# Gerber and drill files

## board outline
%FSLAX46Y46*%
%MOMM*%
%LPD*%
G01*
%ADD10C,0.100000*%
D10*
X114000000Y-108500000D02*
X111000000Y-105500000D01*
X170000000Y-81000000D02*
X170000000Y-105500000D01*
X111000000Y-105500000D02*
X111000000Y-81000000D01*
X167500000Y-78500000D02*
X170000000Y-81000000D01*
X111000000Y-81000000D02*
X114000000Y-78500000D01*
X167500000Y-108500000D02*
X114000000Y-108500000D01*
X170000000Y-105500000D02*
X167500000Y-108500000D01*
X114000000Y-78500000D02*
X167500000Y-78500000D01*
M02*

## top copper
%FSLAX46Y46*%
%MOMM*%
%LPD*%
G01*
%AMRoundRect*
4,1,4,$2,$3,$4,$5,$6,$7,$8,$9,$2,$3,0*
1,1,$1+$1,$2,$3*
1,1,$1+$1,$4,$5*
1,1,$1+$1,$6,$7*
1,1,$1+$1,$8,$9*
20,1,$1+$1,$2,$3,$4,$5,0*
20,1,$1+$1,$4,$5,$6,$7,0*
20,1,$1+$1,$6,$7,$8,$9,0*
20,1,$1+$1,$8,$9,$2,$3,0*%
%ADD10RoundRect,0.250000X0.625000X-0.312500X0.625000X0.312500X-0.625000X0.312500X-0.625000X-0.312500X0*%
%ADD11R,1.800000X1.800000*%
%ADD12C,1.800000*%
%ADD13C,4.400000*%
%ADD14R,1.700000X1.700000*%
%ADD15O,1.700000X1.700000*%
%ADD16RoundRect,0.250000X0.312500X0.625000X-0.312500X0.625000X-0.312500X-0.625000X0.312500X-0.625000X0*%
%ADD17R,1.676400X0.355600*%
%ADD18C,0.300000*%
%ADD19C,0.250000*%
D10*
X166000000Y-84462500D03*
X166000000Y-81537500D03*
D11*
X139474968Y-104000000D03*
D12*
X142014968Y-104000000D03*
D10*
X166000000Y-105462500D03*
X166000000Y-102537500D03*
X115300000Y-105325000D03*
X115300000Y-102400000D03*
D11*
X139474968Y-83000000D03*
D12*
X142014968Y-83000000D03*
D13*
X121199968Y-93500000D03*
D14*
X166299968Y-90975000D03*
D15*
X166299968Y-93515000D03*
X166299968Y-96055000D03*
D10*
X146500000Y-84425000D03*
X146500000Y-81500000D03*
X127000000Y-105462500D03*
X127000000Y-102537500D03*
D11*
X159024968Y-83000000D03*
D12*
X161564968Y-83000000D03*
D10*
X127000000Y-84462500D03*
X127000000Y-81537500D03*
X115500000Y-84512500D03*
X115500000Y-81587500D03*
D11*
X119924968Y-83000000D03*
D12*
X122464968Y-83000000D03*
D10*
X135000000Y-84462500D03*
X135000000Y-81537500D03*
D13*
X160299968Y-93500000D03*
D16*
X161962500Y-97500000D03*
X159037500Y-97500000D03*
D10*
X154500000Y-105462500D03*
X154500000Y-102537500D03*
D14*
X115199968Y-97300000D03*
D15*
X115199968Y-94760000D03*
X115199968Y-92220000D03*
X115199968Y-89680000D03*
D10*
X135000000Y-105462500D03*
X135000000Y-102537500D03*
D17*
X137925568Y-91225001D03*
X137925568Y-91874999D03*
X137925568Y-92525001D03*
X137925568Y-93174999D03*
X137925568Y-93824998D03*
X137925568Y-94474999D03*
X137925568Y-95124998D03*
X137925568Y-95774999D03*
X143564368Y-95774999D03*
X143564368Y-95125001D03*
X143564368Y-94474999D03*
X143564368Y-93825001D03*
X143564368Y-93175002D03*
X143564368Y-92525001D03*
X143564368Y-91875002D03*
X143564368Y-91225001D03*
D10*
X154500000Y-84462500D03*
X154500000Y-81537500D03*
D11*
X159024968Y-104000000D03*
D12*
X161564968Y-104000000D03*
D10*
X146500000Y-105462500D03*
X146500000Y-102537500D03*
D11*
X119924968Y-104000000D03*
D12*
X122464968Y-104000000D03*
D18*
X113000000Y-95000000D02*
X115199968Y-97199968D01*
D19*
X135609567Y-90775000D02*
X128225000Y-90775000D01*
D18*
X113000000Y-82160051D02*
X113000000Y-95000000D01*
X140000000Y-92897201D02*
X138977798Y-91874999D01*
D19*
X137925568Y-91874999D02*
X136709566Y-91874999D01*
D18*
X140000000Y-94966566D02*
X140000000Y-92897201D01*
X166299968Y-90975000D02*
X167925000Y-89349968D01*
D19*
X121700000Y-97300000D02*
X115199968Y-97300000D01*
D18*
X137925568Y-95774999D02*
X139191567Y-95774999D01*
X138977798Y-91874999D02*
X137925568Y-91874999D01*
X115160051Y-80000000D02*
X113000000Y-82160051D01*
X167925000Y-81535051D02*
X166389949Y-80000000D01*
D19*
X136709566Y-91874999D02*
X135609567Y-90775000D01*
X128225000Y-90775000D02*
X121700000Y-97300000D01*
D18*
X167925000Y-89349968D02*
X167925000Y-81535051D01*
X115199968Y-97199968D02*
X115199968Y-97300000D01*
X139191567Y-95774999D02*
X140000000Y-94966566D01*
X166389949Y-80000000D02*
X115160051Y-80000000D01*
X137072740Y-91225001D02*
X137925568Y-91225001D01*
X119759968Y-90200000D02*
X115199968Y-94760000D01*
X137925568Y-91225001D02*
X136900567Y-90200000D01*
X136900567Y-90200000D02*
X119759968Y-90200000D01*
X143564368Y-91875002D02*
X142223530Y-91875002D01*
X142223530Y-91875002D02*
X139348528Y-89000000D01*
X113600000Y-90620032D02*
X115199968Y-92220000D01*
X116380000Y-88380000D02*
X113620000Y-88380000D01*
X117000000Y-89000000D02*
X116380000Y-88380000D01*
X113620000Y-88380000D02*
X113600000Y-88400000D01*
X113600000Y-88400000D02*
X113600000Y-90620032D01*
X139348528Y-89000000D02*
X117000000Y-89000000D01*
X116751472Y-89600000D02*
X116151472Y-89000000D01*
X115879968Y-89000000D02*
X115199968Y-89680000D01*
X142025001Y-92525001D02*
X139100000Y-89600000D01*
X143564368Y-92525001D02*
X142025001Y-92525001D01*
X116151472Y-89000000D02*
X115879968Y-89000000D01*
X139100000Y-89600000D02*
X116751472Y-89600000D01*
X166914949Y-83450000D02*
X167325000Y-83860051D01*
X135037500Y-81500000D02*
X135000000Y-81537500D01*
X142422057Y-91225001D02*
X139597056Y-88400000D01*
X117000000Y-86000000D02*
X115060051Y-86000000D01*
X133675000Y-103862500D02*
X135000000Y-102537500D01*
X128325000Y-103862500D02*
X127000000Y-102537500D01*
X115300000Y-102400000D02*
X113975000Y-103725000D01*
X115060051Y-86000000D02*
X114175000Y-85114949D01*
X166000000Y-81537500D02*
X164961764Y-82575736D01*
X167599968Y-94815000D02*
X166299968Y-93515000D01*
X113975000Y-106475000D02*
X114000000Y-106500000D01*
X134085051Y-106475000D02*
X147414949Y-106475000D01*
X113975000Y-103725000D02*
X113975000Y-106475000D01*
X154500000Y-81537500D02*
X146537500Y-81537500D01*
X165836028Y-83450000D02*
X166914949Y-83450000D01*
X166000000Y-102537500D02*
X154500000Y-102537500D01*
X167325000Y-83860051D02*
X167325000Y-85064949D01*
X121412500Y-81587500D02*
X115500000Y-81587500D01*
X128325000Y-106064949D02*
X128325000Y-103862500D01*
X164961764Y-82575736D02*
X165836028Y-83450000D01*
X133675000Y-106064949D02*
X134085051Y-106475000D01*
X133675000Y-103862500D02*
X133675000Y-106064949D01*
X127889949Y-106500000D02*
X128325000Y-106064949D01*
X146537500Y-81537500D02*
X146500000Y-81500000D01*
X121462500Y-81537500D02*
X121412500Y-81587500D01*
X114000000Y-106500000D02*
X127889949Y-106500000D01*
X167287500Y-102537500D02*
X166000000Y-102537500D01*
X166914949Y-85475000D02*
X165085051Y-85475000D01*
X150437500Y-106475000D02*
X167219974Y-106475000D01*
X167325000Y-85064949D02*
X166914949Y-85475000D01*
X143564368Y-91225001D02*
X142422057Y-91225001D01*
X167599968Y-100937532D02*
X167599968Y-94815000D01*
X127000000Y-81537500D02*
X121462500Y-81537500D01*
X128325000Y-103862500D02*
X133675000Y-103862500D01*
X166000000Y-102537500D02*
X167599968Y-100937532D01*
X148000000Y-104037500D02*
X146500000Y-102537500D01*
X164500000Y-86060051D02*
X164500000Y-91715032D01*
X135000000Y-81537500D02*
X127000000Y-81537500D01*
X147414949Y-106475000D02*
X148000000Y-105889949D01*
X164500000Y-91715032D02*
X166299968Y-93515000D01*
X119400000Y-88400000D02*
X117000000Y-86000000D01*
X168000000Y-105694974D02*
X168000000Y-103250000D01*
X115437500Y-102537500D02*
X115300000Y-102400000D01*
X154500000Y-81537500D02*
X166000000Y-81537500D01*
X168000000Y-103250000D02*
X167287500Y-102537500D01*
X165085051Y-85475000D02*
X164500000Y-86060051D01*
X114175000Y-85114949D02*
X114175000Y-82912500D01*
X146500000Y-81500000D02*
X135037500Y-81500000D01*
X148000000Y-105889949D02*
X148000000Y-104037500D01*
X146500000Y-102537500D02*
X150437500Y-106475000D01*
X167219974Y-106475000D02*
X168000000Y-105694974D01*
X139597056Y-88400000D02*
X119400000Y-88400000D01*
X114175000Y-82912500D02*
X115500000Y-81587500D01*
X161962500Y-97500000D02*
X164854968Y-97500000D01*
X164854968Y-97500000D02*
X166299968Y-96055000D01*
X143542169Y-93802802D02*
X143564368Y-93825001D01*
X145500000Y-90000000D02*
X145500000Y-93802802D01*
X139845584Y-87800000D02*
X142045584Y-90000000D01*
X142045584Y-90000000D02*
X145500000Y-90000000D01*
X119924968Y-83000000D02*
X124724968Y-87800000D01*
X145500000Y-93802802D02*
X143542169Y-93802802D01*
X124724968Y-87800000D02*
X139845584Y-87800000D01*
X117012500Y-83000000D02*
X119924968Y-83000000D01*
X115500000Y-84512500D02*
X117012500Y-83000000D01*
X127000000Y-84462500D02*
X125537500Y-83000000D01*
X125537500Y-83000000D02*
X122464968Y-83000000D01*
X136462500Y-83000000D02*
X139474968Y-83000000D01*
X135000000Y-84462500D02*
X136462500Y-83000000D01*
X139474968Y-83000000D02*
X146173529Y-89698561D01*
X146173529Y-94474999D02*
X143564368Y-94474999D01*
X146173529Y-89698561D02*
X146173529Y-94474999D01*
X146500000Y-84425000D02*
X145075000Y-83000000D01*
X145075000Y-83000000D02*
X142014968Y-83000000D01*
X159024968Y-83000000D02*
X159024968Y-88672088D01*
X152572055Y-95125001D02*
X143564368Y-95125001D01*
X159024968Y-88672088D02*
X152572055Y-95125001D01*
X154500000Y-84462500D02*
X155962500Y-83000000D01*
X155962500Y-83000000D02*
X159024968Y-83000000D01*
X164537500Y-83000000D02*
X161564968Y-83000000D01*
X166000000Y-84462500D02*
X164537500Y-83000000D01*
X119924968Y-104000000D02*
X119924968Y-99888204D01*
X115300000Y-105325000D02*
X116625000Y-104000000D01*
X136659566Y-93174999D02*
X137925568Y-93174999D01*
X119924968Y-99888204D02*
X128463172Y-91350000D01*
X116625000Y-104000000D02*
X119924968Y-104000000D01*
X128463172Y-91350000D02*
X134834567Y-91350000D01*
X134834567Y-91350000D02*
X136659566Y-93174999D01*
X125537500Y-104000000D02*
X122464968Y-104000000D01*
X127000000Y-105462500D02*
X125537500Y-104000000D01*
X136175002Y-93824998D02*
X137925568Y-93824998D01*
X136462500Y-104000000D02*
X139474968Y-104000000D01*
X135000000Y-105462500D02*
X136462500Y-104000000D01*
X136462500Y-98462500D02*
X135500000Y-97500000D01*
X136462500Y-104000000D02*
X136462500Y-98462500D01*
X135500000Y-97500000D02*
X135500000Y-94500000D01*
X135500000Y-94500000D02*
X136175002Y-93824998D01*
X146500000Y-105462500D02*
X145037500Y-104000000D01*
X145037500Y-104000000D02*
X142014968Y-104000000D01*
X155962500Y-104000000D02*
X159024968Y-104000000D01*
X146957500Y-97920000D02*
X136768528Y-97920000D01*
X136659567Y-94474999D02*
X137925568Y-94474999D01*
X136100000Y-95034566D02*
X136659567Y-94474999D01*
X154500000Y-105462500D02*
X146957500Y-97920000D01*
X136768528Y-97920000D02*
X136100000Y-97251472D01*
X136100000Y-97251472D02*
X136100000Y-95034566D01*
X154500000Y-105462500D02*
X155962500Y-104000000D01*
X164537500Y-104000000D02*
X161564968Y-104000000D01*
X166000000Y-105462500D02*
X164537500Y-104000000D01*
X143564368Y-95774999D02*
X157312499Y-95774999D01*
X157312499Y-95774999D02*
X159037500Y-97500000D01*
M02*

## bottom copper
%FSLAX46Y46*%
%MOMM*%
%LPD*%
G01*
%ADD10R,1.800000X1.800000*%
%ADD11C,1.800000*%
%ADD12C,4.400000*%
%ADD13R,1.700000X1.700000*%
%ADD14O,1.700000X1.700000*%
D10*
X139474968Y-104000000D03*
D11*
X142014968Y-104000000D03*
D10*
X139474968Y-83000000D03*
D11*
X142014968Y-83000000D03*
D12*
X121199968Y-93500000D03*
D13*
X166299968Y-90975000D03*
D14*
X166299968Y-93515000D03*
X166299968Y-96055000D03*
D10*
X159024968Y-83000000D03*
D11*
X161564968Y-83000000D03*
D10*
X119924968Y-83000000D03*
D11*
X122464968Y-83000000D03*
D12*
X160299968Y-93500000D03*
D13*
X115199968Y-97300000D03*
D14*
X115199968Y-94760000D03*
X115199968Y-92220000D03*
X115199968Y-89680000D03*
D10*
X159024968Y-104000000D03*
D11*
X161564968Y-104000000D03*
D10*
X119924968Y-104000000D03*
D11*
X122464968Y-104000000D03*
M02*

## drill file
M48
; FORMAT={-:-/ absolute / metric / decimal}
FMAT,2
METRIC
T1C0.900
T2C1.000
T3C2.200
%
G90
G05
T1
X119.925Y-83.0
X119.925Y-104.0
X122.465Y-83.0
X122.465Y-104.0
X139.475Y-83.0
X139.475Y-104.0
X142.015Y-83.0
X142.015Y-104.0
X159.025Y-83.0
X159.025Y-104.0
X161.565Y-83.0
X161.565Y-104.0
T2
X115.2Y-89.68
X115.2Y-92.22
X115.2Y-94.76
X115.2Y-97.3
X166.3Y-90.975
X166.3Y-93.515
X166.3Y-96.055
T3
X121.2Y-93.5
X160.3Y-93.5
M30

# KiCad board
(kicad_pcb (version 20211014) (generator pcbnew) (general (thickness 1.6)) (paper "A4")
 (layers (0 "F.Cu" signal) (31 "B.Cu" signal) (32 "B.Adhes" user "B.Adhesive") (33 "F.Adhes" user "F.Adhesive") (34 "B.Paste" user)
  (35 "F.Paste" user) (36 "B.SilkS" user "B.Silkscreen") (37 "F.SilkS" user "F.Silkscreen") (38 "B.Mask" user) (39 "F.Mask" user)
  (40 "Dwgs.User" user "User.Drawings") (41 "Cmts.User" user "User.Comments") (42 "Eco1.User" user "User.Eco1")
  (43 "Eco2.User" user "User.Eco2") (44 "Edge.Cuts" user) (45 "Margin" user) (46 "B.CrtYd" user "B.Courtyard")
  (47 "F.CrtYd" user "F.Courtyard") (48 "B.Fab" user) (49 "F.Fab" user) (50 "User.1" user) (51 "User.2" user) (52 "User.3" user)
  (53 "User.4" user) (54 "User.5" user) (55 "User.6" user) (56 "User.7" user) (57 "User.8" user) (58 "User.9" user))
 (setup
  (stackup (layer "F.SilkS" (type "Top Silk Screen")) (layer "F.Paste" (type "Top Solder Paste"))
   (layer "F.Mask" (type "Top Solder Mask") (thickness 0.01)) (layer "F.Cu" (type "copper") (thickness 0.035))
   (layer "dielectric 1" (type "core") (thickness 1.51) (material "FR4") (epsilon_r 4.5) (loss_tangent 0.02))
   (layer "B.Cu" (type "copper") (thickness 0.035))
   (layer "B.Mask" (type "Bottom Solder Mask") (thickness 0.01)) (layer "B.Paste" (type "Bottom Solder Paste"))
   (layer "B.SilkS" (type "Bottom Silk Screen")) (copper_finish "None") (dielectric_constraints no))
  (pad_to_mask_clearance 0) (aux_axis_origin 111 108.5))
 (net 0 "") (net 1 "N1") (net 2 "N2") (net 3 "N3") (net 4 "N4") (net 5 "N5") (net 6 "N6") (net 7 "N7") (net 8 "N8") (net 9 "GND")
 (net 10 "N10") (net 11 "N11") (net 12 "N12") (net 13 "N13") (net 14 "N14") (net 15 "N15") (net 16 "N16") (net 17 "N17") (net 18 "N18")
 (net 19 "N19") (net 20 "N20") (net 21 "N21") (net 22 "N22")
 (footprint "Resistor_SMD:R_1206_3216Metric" (layer "F.Cu") (at 166 83 90)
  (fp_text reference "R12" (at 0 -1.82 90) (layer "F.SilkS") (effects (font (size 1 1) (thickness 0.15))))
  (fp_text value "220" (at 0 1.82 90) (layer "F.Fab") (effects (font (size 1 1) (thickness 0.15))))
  (pad "1" smd roundrect (at -1.4625 0 90) (size 1.125 1.75) (layers "F.Cu" "F.Paste" "F.Mask") (roundrect_rratio 0.2222222222) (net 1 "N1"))
  (pad "2" smd roundrect (at 1.4625 0 90) (size 1.125 1.75) (layers "F.Cu" "F.Paste" "F.Mask") (roundrect_rratio 0.2222222222) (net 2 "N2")))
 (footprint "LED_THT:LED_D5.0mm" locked (layer "F.Cu") (at 139.474968 104)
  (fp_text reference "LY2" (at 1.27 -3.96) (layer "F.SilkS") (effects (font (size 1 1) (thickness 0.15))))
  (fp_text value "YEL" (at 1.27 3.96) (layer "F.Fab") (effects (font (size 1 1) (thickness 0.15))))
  (pad "1" thru_hole rect locked (at 0 0) (size 1.8 1.8) (drill 0.9) (layers *.Cu *.Mask) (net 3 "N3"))
  (pad "2" thru_hole circle locked (at 2.54 0) (size 1.8 1.8) (drill 0.9) (layers *.Cu *.Mask) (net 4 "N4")))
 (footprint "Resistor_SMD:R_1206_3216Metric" (layer "F.Cu") (at 166 104 90)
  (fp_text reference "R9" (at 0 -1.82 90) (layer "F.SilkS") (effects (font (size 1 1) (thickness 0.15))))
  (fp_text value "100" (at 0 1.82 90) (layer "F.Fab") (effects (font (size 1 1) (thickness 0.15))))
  (pad "1" smd roundrect (at -1.4625 0 90) (size 1.125 1.75) (layers "F.Cu" "F.Paste" "F.Mask") (roundrect_rratio 0.2222222222) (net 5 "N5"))
  (pad "2" smd roundrect (at 1.4625 0 90) (size 1.125 1.75) (layers "F.Cu" "F.Paste" "F.Mask") (roundrect_rratio 0.2222222222) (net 2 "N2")))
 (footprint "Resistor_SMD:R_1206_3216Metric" (layer "F.Cu") (at 115.3 103.8625 90)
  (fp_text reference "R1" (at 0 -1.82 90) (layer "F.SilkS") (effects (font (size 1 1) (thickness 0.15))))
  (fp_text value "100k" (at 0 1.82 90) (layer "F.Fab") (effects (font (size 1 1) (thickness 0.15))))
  (pad "1" smd roundrect (at -1.4625 0 90) (size 1.125 1.75) (layers "F.Cu" "F.Paste" "F.Mask") (roundrect_rratio 0.2222222222) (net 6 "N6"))
  (pad "2" smd roundrect (at 1.4625 0 90) (size 1.125 1.75) (layers "F.Cu" "F.Paste" "F.Mask") (roundrect_rratio 0.2222222222) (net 2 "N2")))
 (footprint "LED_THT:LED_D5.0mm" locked (layer "F.Cu") (at 139.474968 83)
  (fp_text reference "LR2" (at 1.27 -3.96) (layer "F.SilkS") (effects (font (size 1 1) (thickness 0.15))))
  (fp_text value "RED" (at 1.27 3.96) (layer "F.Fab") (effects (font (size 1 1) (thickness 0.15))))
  (pad "1" thru_hole rect locked (at 0 0) (size 1.8 1.8) (drill 0.9) (layers *.Cu *.Mask) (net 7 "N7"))
  (pad "2" thru_hole circle locked (at 2.54 0) (size 1.8 1.8) (drill 0.9) (layers *.Cu *.Mask) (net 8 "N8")))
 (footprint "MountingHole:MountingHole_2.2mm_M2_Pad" (layer "F.Cu") (at 121.199968 93.5)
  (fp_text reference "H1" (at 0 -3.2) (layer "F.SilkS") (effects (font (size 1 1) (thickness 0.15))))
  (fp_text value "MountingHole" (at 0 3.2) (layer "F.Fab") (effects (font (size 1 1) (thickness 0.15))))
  (pad "1" thru_hole circle (at 0 0) (size 4.4 4.4) (drill 2.2) (layers *.Cu *.Mask)))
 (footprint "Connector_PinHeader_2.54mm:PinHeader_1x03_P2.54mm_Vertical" (layer "F.Cu") (at 166.299968 90.975)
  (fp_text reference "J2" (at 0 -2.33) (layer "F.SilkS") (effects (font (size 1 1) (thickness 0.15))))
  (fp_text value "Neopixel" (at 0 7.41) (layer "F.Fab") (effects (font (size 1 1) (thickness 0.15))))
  (pad "1" thru_hole rect (at 0 0) (size 1.7 1.7) (drill 1) (layers *.Cu *.Mask) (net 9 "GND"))
  (pad "2" thru_hole oval (at 0 2.54) (size 1.7 1.7) (drill 1) (layers *.Cu *.Mask) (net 2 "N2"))
  (pad "3" thru_hole oval (at 0 5.08) (size 1.7 1.7) (drill 1) (layers *.Cu *.Mask) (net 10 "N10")))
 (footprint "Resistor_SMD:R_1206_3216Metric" (layer "F.Cu") (at 146.5 82.9625 90)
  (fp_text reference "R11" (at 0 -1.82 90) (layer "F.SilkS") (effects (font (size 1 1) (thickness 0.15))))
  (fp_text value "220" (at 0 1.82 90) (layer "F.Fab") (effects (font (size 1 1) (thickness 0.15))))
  (pad "1" smd roundrect (at -1.4625 0 90) (size 1.125 1.75) (layers "F.Cu" "F.Paste" "F.Mask") (roundrect_rratio 0.2222222222) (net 8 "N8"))
  (pad "2" smd roundrect (at 1.4625 0 90) (size 1.125 1.75) (layers "F.Cu" "F.Paste" "F.Mask") (roundrect_rratio 0.2222222222) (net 2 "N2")))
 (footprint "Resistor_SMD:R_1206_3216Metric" (layer "F.Cu") (at 127 104 90)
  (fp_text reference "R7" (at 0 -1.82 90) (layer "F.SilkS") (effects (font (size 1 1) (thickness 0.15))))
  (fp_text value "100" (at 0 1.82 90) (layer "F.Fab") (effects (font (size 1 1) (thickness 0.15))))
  (pad "1" smd roundrect (at -1.4625 0 90) (size 1.125 1.75) (layers "F.Cu" "F.Paste" "F.Mask") (roundrect_rratio 0.2222222222)
   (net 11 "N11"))
  (pad "2" smd roundrect (at 1.4625 0 90) (size 1.125 1.75) (layers "F.Cu" "F.Paste" "F.Mask") (roundrect_rratio 0.2222222222) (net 2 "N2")))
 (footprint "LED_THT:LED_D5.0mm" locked (layer "F.Cu") (at 159.024968 83)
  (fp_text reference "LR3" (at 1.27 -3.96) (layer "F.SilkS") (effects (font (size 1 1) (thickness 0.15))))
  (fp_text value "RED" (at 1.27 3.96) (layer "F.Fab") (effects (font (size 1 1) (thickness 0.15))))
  (pad "1" thru_hole rect locked (at 0 0) (size 1.8 1.8) (drill 0.9) (layers *.Cu *.Mask) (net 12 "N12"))
  (pad "2" thru_hole circle locked (at 2.54 0) (size 1.8 1.8) (drill 0.9) (layers *.Cu *.Mask) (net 1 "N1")))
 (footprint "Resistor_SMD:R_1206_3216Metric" (layer "F.Cu") (at 127 83 90)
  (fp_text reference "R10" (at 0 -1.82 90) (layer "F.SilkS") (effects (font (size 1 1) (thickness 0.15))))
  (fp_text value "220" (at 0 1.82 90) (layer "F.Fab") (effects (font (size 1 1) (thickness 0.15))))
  (pad "1" smd roundrect (at -1.4625 0 90) (size 1.125 1.75) (layers "F.Cu" "F.Paste" "F.Mask") (roundrect_rratio 0.2222222222)
   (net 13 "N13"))
  (pad "2" smd roundrect (at 1.4625 0 90) (size 1.125 1.75) (layers "F.Cu" "F.Paste" "F.Mask") (roundrect_rratio 0.2222222222) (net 2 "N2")))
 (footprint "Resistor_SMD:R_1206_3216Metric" (layer "F.Cu") (at 115.5 83.05 90)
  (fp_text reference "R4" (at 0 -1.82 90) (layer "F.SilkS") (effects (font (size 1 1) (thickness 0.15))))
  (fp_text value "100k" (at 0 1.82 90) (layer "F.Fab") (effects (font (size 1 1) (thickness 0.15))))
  (pad "1" smd roundrect (at -1.4625 0 90) (size 1.125 1.75) (layers "F.Cu" "F.Paste" "F.Mask") (roundrect_rratio 0.2222222222)
   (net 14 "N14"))
  (pad "2" smd roundrect (at 1.4625 0 90) (size 1.125 1.75) (layers "F.Cu" "F.Paste" "F.Mask") (roundrect_rratio 0.2222222222) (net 2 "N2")))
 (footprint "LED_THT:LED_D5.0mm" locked (layer "F.Cu") (at 119.924968 83)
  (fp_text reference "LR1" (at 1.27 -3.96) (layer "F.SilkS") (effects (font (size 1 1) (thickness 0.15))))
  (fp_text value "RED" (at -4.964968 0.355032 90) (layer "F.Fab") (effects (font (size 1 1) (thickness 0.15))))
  (pad "1" thru_hole rect locked (at 0 0) (size 1.8 1.8) (drill 0.9) (layers *.Cu *.Mask) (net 14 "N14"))
  (pad "2" thru_hole circle locked (at 2.54 0) (size 1.8 1.8) (drill 0.9) (layers *.Cu *.Mask) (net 13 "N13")))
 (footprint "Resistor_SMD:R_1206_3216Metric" (layer "F.Cu") (at 135 83 90)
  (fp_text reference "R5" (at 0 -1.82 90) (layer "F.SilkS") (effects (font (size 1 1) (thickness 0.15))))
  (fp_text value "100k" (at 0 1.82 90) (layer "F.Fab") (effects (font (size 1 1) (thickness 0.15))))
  (pad "1" smd roundrect (at -1.4625 0 90) (size 1.125 1.75) (layers "F.Cu" "F.Paste" "F.Mask") (roundrect_rratio 0.2222222222) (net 7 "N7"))
  (pad "2" smd roundrect (at 1.4625 0 90) (size 1.125 1.75) (layers "F.Cu" "F.Paste" "F.Mask") (roundrect_rratio 0.2222222222) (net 2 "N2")))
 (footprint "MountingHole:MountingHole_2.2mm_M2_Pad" (layer "F.Cu") (at 160.299968 93.5)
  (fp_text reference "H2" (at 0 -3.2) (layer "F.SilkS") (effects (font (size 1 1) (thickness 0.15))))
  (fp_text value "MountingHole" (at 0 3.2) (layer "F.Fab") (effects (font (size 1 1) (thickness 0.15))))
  (pad "1" thru_hole circle (at 0 0) (size 4.4 4.4) (drill 2.2) (layers *.Cu *.Mask)))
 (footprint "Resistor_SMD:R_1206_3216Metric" (layer "F.Cu") (at 160.5 97.5 180)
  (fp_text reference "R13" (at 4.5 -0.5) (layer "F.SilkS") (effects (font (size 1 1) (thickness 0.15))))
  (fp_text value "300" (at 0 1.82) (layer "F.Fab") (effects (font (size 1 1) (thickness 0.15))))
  (pad "1" smd roundrect (at -1.4625 0 180) (size 1.125 1.75) (layers "F.Cu" "F.Paste" "F.Mask") (roundrect_rratio 0.2222222222)
   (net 10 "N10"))
  (pad "2" smd roundrect (at 1.4625 0 180) (size 1.125 1.75) (layers "F.Cu" "F.Paste" "F.Mask") (roundrect_rratio 0.2222222222)
   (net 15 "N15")))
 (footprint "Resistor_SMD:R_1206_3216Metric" (layer "F.Cu") (at 154.5 104 90)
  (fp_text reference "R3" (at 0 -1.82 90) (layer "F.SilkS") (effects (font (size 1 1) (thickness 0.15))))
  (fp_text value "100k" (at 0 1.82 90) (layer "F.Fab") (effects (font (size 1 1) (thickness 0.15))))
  (pad "1" smd roundrect (at -1.4625 0 90) (size 1.125 1.75) (layers "F.Cu" "F.Paste" "F.Mask") (roundrect_rratio 0.2222222222)
   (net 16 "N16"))
  (pad "2" smd roundrect (at 1.4625 0 90) (size 1.125 1.75) (layers "F.Cu" "F.Paste" "F.Mask") (roundrect_rratio 0.2222222222) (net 2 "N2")))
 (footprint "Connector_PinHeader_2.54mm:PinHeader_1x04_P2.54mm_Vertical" (layer "F.Cu") (at 115.199968 97.3 180)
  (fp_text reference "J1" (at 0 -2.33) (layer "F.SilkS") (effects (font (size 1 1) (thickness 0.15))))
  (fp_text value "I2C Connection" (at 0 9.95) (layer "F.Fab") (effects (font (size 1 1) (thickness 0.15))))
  (pad "1" thru_hole rect (at 0 0 180) (size 1.7 1.7) (drill 1) (layers *.Cu *.Mask) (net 9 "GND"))
  (pad "2" thru_hole oval (at 0 2.54 180) (size 1.7 1.7) (drill 1) (layers *.Cu *.Mask) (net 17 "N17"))
  (pad "3" thru_hole oval (at 0 5.08 180) (size 1.7 1.7) (drill 1) (layers *.Cu *.Mask) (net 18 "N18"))
  (pad "4" thru_hole oval (at 0 7.62 180) (size 1.7 1.7) (drill 1) (layers *.Cu *.Mask) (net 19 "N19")))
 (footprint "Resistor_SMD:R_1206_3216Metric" (layer "F.Cu") (at 135 104 90)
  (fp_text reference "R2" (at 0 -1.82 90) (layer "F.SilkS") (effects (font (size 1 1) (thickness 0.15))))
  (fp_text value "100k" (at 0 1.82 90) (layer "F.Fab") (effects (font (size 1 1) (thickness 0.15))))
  (pad "1" smd roundrect (at -1.4625 0 90) (size 1.125 1.75) (layers "F.Cu" "F.Paste" "F.Mask") (roundrect_rratio 0.2222222222) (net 3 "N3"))
  (pad "2" smd roundrect (at 1.4625 0 90) (size 1.125 1.75) (layers "F.Cu" "F.Paste" "F.Mask") (roundrect_rratio 0.2222222222) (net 2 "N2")))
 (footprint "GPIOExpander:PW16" (layer "F.Cu") (at 140.744968 93.5)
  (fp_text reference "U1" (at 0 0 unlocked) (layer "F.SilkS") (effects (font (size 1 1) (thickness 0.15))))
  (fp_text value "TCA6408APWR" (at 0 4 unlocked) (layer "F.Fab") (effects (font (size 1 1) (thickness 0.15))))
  (pad "1" smd rect (at -2.8194 -2.274999) (size 1.6764 0.3556) (layers "F.Cu" "F.Paste" "F.Mask") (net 17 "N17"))
  (pad "2" smd rect (at -2.8194 -1.625001) (size 1.6764 0.3556) (layers "F.Cu" "F.Paste" "F.Mask") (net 9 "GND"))
  (pad "3" smd rect (at -2.8194 -0.974999) (size 1.6764 0.3556) (layers "F.Cu" "F.Paste" "F.Mask") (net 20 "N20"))
  (pad "4" smd rect (at -2.8194 -0.325001) (size 1.6764 0.3556) (layers "F.Cu" "F.Paste" "F.Mask") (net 6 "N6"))
  (pad "5" smd rect (at -2.8194 0.324998) (size 1.6764 0.3556) (layers "F.Cu" "F.Paste" "F.Mask") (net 3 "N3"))
  (pad "6" smd rect (at -2.8194 0.974999) (size 1.6764 0.3556) (layers "F.Cu" "F.Paste" "F.Mask") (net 16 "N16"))
  (pad "7" smd rect (at -2.8194 1.624998) (size 1.6764 0.3556) (layers "F.Cu" "F.Paste" "F.Mask") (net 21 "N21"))
  (pad "8" smd rect (at -2.8194 2.274999) (size 1.6764 0.3556) (layers "F.Cu" "F.Paste" "F.Mask") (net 9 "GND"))
  (pad "9" smd rect (at 2.8194 2.274999) (size 1.6764 0.3556) (layers "F.Cu" "F.Paste" "F.Mask") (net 15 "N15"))
  (pad "10" smd rect (at 2.8194 1.625001) (size 1.6764 0.3556) (layers "F.Cu" "F.Paste" "F.Mask") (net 12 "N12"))
  (pad "11" smd rect (at 2.8194 0.974999) (size 1.6764 0.3556) (layers "F.Cu" "F.Paste" "F.Mask") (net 7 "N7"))
  (pad "12" smd rect (at 2.8194 0.325001) (size 1.6764 0.3556) (layers "F.Cu" "F.Paste" "F.Mask") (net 14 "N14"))
  (pad "13" smd rect (at 2.8194 -0.324998) (size 1.6764 0.3556) (layers "F.Cu" "F.Paste" "F.Mask") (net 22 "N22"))
  (pad "14" smd rect (at 2.8194 -0.974999) (size 1.6764 0.3556) (layers "F.Cu" "F.Paste" "F.Mask") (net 19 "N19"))
  (pad "15" smd rect (at 2.8194 -1.624998) (size 1.6764 0.3556) (layers "F.Cu" "F.Paste" "F.Mask") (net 18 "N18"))
  (pad "16" smd rect (at 2.8194 -2.274999) (size 1.6764 0.3556) (layers "F.Cu" "F.Paste" "F.Mask") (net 2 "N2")))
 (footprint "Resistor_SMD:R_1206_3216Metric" (layer "F.Cu") (at 154.5 83 90)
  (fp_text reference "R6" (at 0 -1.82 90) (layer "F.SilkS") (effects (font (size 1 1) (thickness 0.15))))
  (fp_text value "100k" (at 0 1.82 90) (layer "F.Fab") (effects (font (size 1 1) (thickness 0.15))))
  (pad "1" smd roundrect (at -1.4625 0 90) (size 1.125 1.75) (layers "F.Cu" "F.Paste" "F.Mask") (roundrect_rratio 0.2222222222)
   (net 12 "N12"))
  (pad "2" smd roundrect (at 1.4625 0 90) (size 1.125 1.75) (layers "F.Cu" "F.Paste" "F.Mask") (roundrect_rratio 0.2222222222) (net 2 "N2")))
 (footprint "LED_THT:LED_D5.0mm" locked (layer "F.Cu") (at 159.024968 104)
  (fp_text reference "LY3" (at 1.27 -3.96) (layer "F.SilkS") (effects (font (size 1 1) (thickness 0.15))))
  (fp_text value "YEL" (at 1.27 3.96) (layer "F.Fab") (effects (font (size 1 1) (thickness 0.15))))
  (pad "1" thru_hole rect locked (at 0 0) (size 1.8 1.8) (drill 0.9) (layers *.Cu *.Mask) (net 16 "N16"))
  (pad "2" thru_hole circle locked (at 2.54 0) (size 1.8 1.8) (drill 0.9) (layers *.Cu *.Mask) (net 5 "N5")))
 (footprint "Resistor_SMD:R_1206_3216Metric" (layer "F.Cu") (at 146.5 104 90)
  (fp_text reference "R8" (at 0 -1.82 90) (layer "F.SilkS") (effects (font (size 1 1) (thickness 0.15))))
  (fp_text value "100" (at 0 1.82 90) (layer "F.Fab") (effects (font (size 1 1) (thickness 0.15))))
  (pad "1" smd roundrect (at -1.4625 0 90) (size 1.125 1.75) (layers "F.Cu" "F.Paste" "F.Mask") (roundrect_rratio 0.2222222222) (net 4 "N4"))
  (pad "2" smd roundrect (at 1.4625 0 90) (size 1.125 1.75) (layers "F.Cu" "F.Paste" "F.Mask") (roundrect_rratio 0.2222222222) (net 2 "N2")))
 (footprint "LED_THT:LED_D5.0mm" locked (layer "F.Cu") (at 119.924968 104)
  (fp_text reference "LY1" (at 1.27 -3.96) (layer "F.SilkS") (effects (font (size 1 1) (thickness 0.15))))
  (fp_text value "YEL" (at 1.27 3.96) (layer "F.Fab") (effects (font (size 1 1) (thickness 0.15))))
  (pad "1" thru_hole rect locked (at 0 0) (size 1.8 1.8) (drill 0.9) (layers *.Cu *.Mask) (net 6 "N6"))
  (pad "2" thru_hole circle locked (at 2.54 0) (size 1.8 1.8) (drill 0.9) (layers *.Cu *.Mask) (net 11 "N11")))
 (gr_line (start 114 108.5) (end 111 105.5) (layer "Edge.Cuts") (width 0.1))
 (gr_line (start 170 81) (end 170 105.5) (layer "Edge.Cuts") (width 0.1))
 (gr_line (start 111 105.5) (end 111 81) (layer "Edge.Cuts") (width 0.1))
 (gr_line (start 167.5 78.5) (end 170 81) (layer "Edge.Cuts") (width 0.1))
 (gr_line (start 111 81) (end 114 78.5) (layer "Edge.Cuts") (width 0.1))
 (gr_line (start 167.5 108.5) (end 114 108.5) (layer "Edge.Cuts") (width 0.1))
 (gr_line (start 170 105.5) (end 167.5 108.5) (layer "Edge.Cuts") (width 0.1))
 (gr_line (start 114 78.5) (end 167.5 78.5) (layer "Edge.Cuts") (width 0.1))
 (segment (start 113 95) (end 115.199968 97.199968) (width 0.3) (layer "F.Cu") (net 9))
 (segment (start 135.609567 90.775) (end 128.225 90.775) (width 0.25) (layer "F.Cu") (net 9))
 (segment (start 113 82.160051) (end 113 95) (width 0.3) (layer "F.Cu") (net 9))
 (segment (start 140 92.897201) (end 138.977798 91.874999) (width 0.3) (layer "F.Cu") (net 9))
 (segment (start 137.925568 91.874999) (end 136.709566 91.874999) (width 0.25) (layer "F.Cu") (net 9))
 (segment (start 140 94.966566) (end 140 92.897201) (width 0.3) (layer "F.Cu") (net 9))
 (segment (start 166.299968 90.975) (end 167.925 89.349968) (width 0.3) (layer "F.Cu") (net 9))
 (segment (start 121.7 97.3) (end 115.199968 97.3) (width 0.25) (layer "F.Cu") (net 9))
 (segment (start 137.925568 95.774999) (end 139.191567 95.774999) (width 0.3) (layer "F.Cu") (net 9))
 (segment (start 138.977798 91.874999) (end 137.925568 91.874999) (width 0.3) (layer "F.Cu") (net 9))
 (segment (start 115.160051 80) (end 113 82.160051) (width 0.3) (layer "F.Cu") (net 9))
 (segment (start 167.925 81.535051) (end 166.389949 80) (width 0.3) (layer "F.Cu") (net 9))
 (segment (start 136.709566 91.874999) (end 135.609567 90.775) (width 0.25) (layer "F.Cu") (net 9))
 (segment (start 128.225 90.775) (end 121.7 97.3) (width 0.25) (layer "F.Cu") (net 9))
 (segment (start 167.925 89.349968) (end 167.925 81.535051) (width 0.3) (layer "F.Cu") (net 9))
 (segment (start 115.199968 97.199968) (end 115.199968 97.3) (width 0.3) (layer "F.Cu") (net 9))
 (segment (start 139.191567 95.774999) (end 140 94.966566) (width 0.3) (layer "F.Cu") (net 9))
 (segment (start 166.389949 80) (end 115.160051 80) (width 0.3) (layer "F.Cu") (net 9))
 (segment (start 137.07274 91.225001) (end 137.925568 91.225001) (width 0.3) (layer "F.Cu") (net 17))
 (segment (start 119.759968 90.2) (end 115.199968 94.76) (width 0.3) (layer "F.Cu") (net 17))
 (segment (start 137.925568 91.225001) (end 136.900567 90.2) (width 0.3) (layer "F.Cu") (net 17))
 (segment (start 136.900567 90.2) (end 119.759968 90.2) (width 0.3) (layer "F.Cu") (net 17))
 (segment (start 143.564368 91.875002) (end 142.22353 91.875002) (width 0.3) (layer "F.Cu") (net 18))
 (segment (start 142.22353 91.875002) (end 139.348528 89) (width 0.3) (layer "F.Cu") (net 18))
 (segment (start 113.6 90.620032) (end 115.199968 92.22) (width 0.3) (layer "F.Cu") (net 18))
 (segment (start 116.38 88.38) (end 113.62 88.38) (width 0.3) (layer "F.Cu") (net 18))
 (segment (start 117 89) (end 116.38 88.38) (width 0.3) (layer "F.Cu") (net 18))
 (segment (start 113.62 88.38) (end 113.6 88.4) (width 0.3) (layer "F.Cu") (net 18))
 (segment (start 113.6 88.4) (end 113.6 90.620032) (width 0.3) (layer "F.Cu") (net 18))
 (segment (start 139.348528 89) (end 117 89) (width 0.3) (layer "F.Cu") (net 18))
 (segment (start 116.751472 89.6) (end 116.151472 89) (width 0.3) (layer "F.Cu") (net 19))
 (segment (start 115.879968 89) (end 115.199968 89.68) (width 0.3) (layer "F.Cu") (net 19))
 (segment (start 142.025001 92.525001) (end 139.1 89.6) (width 0.3) (layer "F.Cu") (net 19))
 (segment (start 143.564368 92.525001) (end 142.025001 92.525001) (width 0.3) (layer "F.Cu") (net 19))
 (segment (start 116.151472 89) (end 115.879968 89) (width 0.3) (layer "F.Cu") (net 19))
 (segment (start 139.1 89.6) (end 116.751472 89.6) (width 0.3) (layer "F.Cu") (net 19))
 (segment (start 166.914949 83.45) (end 167.325 83.860051) (width 0.3) (layer "F.Cu") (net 2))
 (segment (start 135.0375 81.5) (end 135 81.5375) (width 0.3) (layer "F.Cu") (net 2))
 (segment (start 142.422057 91.225001) (end 139.597056 88.4) (width 0.3) (layer "F.Cu") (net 2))
 (segment (start 117 86) (end 115.060051 86) (width 0.3) (layer "F.Cu") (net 2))
 (segment (start 133.675 103.8625) (end 135 102.5375) (width 0.3) (layer "F.Cu") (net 2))
 (segment (start 128.325 103.8625) (end 127 102.5375) (width 0.3) (layer "F.Cu") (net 2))
 (segment (start 115.3 102.4) (end 113.975 103.725) (width 0.3) (layer "F.Cu") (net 2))
 (segment (start 115.060051 86) (end 114.175 85.114949) (width 0.3) (layer "F.Cu") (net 2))
 (segment (start 166 81.5375) (end 164.961764 82.575736) (width 0.3) (layer "F.Cu") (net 2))
 (segment (start 167.599968 94.815) (end 166.299968 93.515) (width 0.3) (layer "F.Cu") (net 2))
 (segment (start 113.975 106.475) (end 114 106.5) (width 0.3) (layer "F.Cu") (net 2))
 (segment (start 134.085051 106.475) (end 147.414949 106.475) (width 0.3) (layer "F.Cu") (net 2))
 (segment (start 113.975 103.725) (end 113.975 106.475) (width 0.3) (layer "F.Cu") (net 2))
 (segment (start 154.5 81.5375) (end 146.5375 81.5375) (width 0.3) (layer "F.Cu") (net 2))
 (segment (start 165.836028 83.45) (end 166.914949 83.45) (width 0.3) (layer "F.Cu") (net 2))
 (segment (start 166 102.5375) (end 154.5 102.5375) (width 0.3) (layer "F.Cu") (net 2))
 (segment (start 167.325 83.860051) (end 167.325 85.064949) (width 0.3) (layer "F.Cu") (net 2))
 (segment (start 121.4125 81.5875) (end 115.5 81.5875) (width 0.3) (layer "F.Cu") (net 2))
 (segment (start 128.325 106.064949) (end 128.325 103.8625) (width 0.3) (layer "F.Cu") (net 2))
 (segment (start 164.961764 82.575736) (end 165.836028 83.45) (width 0.3) (layer "F.Cu") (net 2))
 (segment (start 133.675 106.064949) (end 134.085051 106.475) (width 0.3) (layer "F.Cu") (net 2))
 (segment (start 133.675 103.8625) (end 133.675 106.064949) (width 0.3) (layer "F.Cu") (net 2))
 (segment (start 127.889949 106.5) (end 128.325 106.064949) (width 0.3) (layer "F.Cu") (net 2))
 (segment (start 146.5375 81.5375) (end 146.5 81.5) (width 0.3) (layer "F.Cu") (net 2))
 (segment (start 121.4625 81.5375) (end 121.4125 81.5875) (width 0.3) (layer "F.Cu") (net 2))
 (segment (start 114 106.5) (end 127.889949 106.5) (width 0.3) (layer "F.Cu") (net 2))
 (segment (start 167.2875 102.5375) (end 166 102.5375) (width 0.3) (layer "F.Cu") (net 2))
 (segment (start 166.914949 85.475) (end 165.085051 85.475) (width 0.3) (layer "F.Cu") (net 2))
 (segment (start 150.4375 106.475) (end 167.219974 106.475) (width 0.3) (layer "F.Cu") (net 2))
 (segment (start 167.325 85.064949) (end 166.914949 85.475) (width 0.3) (layer "F.Cu") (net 2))
 (segment (start 143.564368 91.225001) (end 142.422057 91.225001) (width 0.3) (layer "F.Cu") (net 2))
 (segment (start 167.599968 100.937532) (end 167.599968 94.815) (width 0.3) (layer "F.Cu") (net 2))
 (segment (start 127 81.5375) (end 121.4625 81.5375) (width 0.3) (layer "F.Cu") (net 2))
 (segment (start 128.325 103.8625) (end 133.675 103.8625) (width 0.3) (layer "F.Cu") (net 2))
 (segment (start 166 102.5375) (end 167.599968 100.937532) (width 0.3) (layer "F.Cu") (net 2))
 (segment (start 148 104.0375) (end 146.5 102.5375) (width 0.3) (layer "F.Cu") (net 2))
 (segment (start 164.5 86.060051) (end 164.5 91.715032) (width 0.3) (layer "F.Cu") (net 2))
 (segment (start 135 81.5375) (end 127 81.5375) (width 0.3) (layer "F.Cu") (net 2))
 (segment (start 147.414949 106.475) (end 148 105.889949) (width 0.3) (layer "F.Cu") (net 2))
 (segment (start 164.5 91.715032) (end 166.299968 93.515) (width 0.3) (layer "F.Cu") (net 2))
 (segment (start 119.4 88.4) (end 117 86) (width 0.3) (layer "F.Cu") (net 2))
 (segment (start 168 105.694974) (end 168 103.25) (width 0.3) (layer "F.Cu") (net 2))
 (segment (start 115.4375 102.5375) (end 115.3 102.4) (width 0.3) (layer "F.Cu") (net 2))
 (segment (start 154.5 81.5375) (end 166 81.5375) (width 0.3) (layer "F.Cu") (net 2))
 (segment (start 168 103.25) (end 167.2875 102.5375) (width 0.3) (layer "F.Cu") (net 2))
 (segment (start 165.085051 85.475) (end 164.5 86.060051) (width 0.3) (layer "F.Cu") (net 2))
 (segment (start 114.175 85.114949) (end 114.175 82.9125) (width 0.3) (layer "F.Cu") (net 2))
 (segment (start 146.5 81.5) (end 135.0375 81.5) (width 0.3) (layer "F.Cu") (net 2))
 (segment (start 148 105.889949) (end 148 104.0375) (width 0.3) (layer "F.Cu") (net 2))
 (segment (start 146.5 102.5375) (end 150.4375 106.475) (width 0.3) (layer "F.Cu") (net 2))
 (segment (start 167.219974 106.475) (end 168 105.694974) (width 0.3) (layer "F.Cu") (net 2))
 (segment (start 139.597056 88.4) (end 119.4 88.4) (width 0.3) (layer "F.Cu") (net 2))
 (segment (start 114.175 82.9125) (end 115.5 81.5875) (width 0.3) (layer "F.Cu") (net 2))
 (segment (start 161.9625 97.5) (end 164.854968 97.5) (width 0.3) (layer "F.Cu") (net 10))
 (segment (start 164.854968 97.5) (end 166.299968 96.055) (width 0.3) (layer "F.Cu") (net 10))
 (segment (start 143.542169 93.802802) (end 143.564368 93.825001) (width 0.3) (layer "F.Cu") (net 14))
 (segment (start 145.5 90) (end 145.5 93.802802) (width 0.3) (layer "F.Cu") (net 14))
 (segment (start 139.845584 87.8) (end 142.045584 90) (width 0.3) (layer "F.Cu") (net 14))
 (segment (start 142.045584 90) (end 145.5 90) (width 0.3) (layer "F.Cu") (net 14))
 (segment (start 119.924968 83) (end 124.724968 87.8) (width 0.3) (layer "F.Cu") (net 14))
 (segment (start 145.5 93.802802) (end 143.542169 93.802802) (width 0.3) (layer "F.Cu") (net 14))
 (segment (start 124.724968 87.8) (end 139.845584 87.8) (width 0.3) (layer "F.Cu") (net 14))
 (segment (start 117.0125 83) (end 119.924968 83) (width 0.3) (layer "F.Cu") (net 14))
 (segment (start 115.5 84.5125) (end 117.0125 83) (width 0.3) (layer "F.Cu") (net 14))
 (segment (start 127 84.4625) (end 125.5375 83) (width 0.3) (layer "F.Cu") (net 13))
 (segment (start 125.5375 83) (end 122.464968 83) (width 0.3) (layer "F.Cu") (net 13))
 (segment (start 136.4625 83) (end 139.474968 83) (width 0.3) (layer "F.Cu") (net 7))
 (segment (start 135 84.4625) (end 136.4625 83) (width 0.3) (layer "F.Cu") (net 7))
 (segment (start 139.474968 83) (end 146.173529 89.698561) (width 0.3) (layer "F.Cu") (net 7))
 (segment (start 146.173529 94.474999) (end 143.564368 94.474999) (width 0.3) (layer "F.Cu") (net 7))
 (segment (start 146.173529 89.698561) (end 146.173529 94.474999) (width 0.3) (layer "F.Cu") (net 7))
 (segment (start 146.5 84.425) (end 145.075 83) (width 0.3) (layer "F.Cu") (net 8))
 (segment (start 145.075 83) (end 142.014968 83) (width 0.3) (layer "F.Cu") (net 8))
 (segment (start 159.024968 83) (end 159.024968 88.672088) (width 0.3) (layer "F.Cu") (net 12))
 (segment (start 152.572055 95.125001) (end 143.564368 95.125001) (width 0.3) (layer "F.Cu") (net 12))
 (segment (start 159.024968 88.672088) (end 152.572055 95.125001) (width 0.3) (layer "F.Cu") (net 12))
 (segment (start 154.5 84.4625) (end 155.9625 83) (width 0.3) (layer "F.Cu") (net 12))
 (segment (start 155.9625 83) (end 159.024968 83) (width 0.3) (layer "F.Cu") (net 12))
 (segment (start 164.5375 83) (end 161.564968 83) (width 0.3) (layer "F.Cu") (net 1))
 (segment (start 166 84.4625) (end 164.5375 83) (width 0.3) (layer "F.Cu") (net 1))
 (segment (start 119.924968 104) (end 119.924968 99.888204) (width 0.3) (layer "F.Cu") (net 6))
 (segment (start 115.3 105.325) (end 116.625 104) (width 0.3) (layer "F.Cu") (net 6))
 (segment (start 136.659566 93.174999) (end 137.925568 93.174999) (width 0.3) (layer "F.Cu") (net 6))
 (segment (start 119.924968 99.888204) (end 128.463172 91.35) (width 0.3) (layer "F.Cu") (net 6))
 (segment (start 116.625 104) (end 119.924968 104) (width 0.3) (layer "F.Cu") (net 6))
 (segment (start 128.463172 91.35) (end 134.834567 91.35) (width 0.3) (layer "F.Cu") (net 6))
 (segment (start 134.834567 91.35) (end 136.659566 93.174999) (width 0.3) (layer "F.Cu") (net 6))
 (segment (start 125.5375 104) (end 122.464968 104) (width 0.3) (layer "F.Cu") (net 11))
 (segment (start 127 105.4625) (end 125.5375 104) (width 0.3) (layer "F.Cu") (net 11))
 (segment (start 136.175002 93.824998) (end 137.925568 93.824998) (width 0.3) (layer "F.Cu") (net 3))
 (segment (start 136.4625 104) (end 139.474968 104) (width 0.3) (layer "F.Cu") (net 3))
 (segment (start 135 105.4625) (end 136.4625 104) (width 0.3) (layer "F.Cu") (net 3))
 (segment (start 136.4625 98.4625) (end 135.5 97.5) (width 0.3) (layer "F.Cu") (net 3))
 (segment (start 136.4625 104) (end 136.4625 98.4625) (width 0.3) (layer "F.Cu") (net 3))
 (segment (start 135.5 97.5) (end 135.5 94.5) (width 0.3) (layer "F.Cu") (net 3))
 (segment (start 135.5 94.5) (end 136.175002 93.824998) (width 0.3) (layer "F.Cu") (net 3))
 (segment (start 146.5 105.4625) (end 145.0375 104) (width 0.3) (layer "F.Cu") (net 4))
 (segment (start 145.0375 104) (end 142.014968 104) (width 0.3) (layer "F.Cu") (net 4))
 (segment (start 155.9625 104) (end 159.024968 104) (width 0.3) (layer "F.Cu") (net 16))
 (segment (start 146.9575 97.92) (end 136.768528 97.92) (width 0.3) (layer "F.Cu") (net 16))
 (segment (start 136.659567 94.474999) (end 137.925568 94.474999) (width 0.3) (layer "F.Cu") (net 16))
 (segment (start 136.1 95.034566) (end 136.659567 94.474999) (width 0.3) (layer "F.Cu") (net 16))
 (segment (start 154.5 105.4625) (end 146.9575 97.92) (width 0.3) (layer "F.Cu") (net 16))
 (segment (start 136.768528 97.92) (end 136.1 97.251472) (width 0.3) (layer "F.Cu") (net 16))
 (segment (start 136.1 97.251472) (end 136.1 95.034566) (width 0.3) (layer "F.Cu") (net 16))
 (segment (start 154.5 105.4625) (end 155.9625 104) (width 0.3) (layer "F.Cu") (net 16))
 (segment (start 164.5375 104) (end 161.564968 104) (width 0.3) (layer "F.Cu") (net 5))
 (segment (start 166 105.4625) (end 164.5375 104) (width 0.3) (layer "F.Cu") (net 5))
 (segment (start 143.564368 95.774999) (end 157.312499 95.774999) (width 0.3) (layer "F.Cu") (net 15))
 (segment (start 157.312499 95.774999) (end 159.0375 97.5) (width 0.3) (layer "F.Cu") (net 15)))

